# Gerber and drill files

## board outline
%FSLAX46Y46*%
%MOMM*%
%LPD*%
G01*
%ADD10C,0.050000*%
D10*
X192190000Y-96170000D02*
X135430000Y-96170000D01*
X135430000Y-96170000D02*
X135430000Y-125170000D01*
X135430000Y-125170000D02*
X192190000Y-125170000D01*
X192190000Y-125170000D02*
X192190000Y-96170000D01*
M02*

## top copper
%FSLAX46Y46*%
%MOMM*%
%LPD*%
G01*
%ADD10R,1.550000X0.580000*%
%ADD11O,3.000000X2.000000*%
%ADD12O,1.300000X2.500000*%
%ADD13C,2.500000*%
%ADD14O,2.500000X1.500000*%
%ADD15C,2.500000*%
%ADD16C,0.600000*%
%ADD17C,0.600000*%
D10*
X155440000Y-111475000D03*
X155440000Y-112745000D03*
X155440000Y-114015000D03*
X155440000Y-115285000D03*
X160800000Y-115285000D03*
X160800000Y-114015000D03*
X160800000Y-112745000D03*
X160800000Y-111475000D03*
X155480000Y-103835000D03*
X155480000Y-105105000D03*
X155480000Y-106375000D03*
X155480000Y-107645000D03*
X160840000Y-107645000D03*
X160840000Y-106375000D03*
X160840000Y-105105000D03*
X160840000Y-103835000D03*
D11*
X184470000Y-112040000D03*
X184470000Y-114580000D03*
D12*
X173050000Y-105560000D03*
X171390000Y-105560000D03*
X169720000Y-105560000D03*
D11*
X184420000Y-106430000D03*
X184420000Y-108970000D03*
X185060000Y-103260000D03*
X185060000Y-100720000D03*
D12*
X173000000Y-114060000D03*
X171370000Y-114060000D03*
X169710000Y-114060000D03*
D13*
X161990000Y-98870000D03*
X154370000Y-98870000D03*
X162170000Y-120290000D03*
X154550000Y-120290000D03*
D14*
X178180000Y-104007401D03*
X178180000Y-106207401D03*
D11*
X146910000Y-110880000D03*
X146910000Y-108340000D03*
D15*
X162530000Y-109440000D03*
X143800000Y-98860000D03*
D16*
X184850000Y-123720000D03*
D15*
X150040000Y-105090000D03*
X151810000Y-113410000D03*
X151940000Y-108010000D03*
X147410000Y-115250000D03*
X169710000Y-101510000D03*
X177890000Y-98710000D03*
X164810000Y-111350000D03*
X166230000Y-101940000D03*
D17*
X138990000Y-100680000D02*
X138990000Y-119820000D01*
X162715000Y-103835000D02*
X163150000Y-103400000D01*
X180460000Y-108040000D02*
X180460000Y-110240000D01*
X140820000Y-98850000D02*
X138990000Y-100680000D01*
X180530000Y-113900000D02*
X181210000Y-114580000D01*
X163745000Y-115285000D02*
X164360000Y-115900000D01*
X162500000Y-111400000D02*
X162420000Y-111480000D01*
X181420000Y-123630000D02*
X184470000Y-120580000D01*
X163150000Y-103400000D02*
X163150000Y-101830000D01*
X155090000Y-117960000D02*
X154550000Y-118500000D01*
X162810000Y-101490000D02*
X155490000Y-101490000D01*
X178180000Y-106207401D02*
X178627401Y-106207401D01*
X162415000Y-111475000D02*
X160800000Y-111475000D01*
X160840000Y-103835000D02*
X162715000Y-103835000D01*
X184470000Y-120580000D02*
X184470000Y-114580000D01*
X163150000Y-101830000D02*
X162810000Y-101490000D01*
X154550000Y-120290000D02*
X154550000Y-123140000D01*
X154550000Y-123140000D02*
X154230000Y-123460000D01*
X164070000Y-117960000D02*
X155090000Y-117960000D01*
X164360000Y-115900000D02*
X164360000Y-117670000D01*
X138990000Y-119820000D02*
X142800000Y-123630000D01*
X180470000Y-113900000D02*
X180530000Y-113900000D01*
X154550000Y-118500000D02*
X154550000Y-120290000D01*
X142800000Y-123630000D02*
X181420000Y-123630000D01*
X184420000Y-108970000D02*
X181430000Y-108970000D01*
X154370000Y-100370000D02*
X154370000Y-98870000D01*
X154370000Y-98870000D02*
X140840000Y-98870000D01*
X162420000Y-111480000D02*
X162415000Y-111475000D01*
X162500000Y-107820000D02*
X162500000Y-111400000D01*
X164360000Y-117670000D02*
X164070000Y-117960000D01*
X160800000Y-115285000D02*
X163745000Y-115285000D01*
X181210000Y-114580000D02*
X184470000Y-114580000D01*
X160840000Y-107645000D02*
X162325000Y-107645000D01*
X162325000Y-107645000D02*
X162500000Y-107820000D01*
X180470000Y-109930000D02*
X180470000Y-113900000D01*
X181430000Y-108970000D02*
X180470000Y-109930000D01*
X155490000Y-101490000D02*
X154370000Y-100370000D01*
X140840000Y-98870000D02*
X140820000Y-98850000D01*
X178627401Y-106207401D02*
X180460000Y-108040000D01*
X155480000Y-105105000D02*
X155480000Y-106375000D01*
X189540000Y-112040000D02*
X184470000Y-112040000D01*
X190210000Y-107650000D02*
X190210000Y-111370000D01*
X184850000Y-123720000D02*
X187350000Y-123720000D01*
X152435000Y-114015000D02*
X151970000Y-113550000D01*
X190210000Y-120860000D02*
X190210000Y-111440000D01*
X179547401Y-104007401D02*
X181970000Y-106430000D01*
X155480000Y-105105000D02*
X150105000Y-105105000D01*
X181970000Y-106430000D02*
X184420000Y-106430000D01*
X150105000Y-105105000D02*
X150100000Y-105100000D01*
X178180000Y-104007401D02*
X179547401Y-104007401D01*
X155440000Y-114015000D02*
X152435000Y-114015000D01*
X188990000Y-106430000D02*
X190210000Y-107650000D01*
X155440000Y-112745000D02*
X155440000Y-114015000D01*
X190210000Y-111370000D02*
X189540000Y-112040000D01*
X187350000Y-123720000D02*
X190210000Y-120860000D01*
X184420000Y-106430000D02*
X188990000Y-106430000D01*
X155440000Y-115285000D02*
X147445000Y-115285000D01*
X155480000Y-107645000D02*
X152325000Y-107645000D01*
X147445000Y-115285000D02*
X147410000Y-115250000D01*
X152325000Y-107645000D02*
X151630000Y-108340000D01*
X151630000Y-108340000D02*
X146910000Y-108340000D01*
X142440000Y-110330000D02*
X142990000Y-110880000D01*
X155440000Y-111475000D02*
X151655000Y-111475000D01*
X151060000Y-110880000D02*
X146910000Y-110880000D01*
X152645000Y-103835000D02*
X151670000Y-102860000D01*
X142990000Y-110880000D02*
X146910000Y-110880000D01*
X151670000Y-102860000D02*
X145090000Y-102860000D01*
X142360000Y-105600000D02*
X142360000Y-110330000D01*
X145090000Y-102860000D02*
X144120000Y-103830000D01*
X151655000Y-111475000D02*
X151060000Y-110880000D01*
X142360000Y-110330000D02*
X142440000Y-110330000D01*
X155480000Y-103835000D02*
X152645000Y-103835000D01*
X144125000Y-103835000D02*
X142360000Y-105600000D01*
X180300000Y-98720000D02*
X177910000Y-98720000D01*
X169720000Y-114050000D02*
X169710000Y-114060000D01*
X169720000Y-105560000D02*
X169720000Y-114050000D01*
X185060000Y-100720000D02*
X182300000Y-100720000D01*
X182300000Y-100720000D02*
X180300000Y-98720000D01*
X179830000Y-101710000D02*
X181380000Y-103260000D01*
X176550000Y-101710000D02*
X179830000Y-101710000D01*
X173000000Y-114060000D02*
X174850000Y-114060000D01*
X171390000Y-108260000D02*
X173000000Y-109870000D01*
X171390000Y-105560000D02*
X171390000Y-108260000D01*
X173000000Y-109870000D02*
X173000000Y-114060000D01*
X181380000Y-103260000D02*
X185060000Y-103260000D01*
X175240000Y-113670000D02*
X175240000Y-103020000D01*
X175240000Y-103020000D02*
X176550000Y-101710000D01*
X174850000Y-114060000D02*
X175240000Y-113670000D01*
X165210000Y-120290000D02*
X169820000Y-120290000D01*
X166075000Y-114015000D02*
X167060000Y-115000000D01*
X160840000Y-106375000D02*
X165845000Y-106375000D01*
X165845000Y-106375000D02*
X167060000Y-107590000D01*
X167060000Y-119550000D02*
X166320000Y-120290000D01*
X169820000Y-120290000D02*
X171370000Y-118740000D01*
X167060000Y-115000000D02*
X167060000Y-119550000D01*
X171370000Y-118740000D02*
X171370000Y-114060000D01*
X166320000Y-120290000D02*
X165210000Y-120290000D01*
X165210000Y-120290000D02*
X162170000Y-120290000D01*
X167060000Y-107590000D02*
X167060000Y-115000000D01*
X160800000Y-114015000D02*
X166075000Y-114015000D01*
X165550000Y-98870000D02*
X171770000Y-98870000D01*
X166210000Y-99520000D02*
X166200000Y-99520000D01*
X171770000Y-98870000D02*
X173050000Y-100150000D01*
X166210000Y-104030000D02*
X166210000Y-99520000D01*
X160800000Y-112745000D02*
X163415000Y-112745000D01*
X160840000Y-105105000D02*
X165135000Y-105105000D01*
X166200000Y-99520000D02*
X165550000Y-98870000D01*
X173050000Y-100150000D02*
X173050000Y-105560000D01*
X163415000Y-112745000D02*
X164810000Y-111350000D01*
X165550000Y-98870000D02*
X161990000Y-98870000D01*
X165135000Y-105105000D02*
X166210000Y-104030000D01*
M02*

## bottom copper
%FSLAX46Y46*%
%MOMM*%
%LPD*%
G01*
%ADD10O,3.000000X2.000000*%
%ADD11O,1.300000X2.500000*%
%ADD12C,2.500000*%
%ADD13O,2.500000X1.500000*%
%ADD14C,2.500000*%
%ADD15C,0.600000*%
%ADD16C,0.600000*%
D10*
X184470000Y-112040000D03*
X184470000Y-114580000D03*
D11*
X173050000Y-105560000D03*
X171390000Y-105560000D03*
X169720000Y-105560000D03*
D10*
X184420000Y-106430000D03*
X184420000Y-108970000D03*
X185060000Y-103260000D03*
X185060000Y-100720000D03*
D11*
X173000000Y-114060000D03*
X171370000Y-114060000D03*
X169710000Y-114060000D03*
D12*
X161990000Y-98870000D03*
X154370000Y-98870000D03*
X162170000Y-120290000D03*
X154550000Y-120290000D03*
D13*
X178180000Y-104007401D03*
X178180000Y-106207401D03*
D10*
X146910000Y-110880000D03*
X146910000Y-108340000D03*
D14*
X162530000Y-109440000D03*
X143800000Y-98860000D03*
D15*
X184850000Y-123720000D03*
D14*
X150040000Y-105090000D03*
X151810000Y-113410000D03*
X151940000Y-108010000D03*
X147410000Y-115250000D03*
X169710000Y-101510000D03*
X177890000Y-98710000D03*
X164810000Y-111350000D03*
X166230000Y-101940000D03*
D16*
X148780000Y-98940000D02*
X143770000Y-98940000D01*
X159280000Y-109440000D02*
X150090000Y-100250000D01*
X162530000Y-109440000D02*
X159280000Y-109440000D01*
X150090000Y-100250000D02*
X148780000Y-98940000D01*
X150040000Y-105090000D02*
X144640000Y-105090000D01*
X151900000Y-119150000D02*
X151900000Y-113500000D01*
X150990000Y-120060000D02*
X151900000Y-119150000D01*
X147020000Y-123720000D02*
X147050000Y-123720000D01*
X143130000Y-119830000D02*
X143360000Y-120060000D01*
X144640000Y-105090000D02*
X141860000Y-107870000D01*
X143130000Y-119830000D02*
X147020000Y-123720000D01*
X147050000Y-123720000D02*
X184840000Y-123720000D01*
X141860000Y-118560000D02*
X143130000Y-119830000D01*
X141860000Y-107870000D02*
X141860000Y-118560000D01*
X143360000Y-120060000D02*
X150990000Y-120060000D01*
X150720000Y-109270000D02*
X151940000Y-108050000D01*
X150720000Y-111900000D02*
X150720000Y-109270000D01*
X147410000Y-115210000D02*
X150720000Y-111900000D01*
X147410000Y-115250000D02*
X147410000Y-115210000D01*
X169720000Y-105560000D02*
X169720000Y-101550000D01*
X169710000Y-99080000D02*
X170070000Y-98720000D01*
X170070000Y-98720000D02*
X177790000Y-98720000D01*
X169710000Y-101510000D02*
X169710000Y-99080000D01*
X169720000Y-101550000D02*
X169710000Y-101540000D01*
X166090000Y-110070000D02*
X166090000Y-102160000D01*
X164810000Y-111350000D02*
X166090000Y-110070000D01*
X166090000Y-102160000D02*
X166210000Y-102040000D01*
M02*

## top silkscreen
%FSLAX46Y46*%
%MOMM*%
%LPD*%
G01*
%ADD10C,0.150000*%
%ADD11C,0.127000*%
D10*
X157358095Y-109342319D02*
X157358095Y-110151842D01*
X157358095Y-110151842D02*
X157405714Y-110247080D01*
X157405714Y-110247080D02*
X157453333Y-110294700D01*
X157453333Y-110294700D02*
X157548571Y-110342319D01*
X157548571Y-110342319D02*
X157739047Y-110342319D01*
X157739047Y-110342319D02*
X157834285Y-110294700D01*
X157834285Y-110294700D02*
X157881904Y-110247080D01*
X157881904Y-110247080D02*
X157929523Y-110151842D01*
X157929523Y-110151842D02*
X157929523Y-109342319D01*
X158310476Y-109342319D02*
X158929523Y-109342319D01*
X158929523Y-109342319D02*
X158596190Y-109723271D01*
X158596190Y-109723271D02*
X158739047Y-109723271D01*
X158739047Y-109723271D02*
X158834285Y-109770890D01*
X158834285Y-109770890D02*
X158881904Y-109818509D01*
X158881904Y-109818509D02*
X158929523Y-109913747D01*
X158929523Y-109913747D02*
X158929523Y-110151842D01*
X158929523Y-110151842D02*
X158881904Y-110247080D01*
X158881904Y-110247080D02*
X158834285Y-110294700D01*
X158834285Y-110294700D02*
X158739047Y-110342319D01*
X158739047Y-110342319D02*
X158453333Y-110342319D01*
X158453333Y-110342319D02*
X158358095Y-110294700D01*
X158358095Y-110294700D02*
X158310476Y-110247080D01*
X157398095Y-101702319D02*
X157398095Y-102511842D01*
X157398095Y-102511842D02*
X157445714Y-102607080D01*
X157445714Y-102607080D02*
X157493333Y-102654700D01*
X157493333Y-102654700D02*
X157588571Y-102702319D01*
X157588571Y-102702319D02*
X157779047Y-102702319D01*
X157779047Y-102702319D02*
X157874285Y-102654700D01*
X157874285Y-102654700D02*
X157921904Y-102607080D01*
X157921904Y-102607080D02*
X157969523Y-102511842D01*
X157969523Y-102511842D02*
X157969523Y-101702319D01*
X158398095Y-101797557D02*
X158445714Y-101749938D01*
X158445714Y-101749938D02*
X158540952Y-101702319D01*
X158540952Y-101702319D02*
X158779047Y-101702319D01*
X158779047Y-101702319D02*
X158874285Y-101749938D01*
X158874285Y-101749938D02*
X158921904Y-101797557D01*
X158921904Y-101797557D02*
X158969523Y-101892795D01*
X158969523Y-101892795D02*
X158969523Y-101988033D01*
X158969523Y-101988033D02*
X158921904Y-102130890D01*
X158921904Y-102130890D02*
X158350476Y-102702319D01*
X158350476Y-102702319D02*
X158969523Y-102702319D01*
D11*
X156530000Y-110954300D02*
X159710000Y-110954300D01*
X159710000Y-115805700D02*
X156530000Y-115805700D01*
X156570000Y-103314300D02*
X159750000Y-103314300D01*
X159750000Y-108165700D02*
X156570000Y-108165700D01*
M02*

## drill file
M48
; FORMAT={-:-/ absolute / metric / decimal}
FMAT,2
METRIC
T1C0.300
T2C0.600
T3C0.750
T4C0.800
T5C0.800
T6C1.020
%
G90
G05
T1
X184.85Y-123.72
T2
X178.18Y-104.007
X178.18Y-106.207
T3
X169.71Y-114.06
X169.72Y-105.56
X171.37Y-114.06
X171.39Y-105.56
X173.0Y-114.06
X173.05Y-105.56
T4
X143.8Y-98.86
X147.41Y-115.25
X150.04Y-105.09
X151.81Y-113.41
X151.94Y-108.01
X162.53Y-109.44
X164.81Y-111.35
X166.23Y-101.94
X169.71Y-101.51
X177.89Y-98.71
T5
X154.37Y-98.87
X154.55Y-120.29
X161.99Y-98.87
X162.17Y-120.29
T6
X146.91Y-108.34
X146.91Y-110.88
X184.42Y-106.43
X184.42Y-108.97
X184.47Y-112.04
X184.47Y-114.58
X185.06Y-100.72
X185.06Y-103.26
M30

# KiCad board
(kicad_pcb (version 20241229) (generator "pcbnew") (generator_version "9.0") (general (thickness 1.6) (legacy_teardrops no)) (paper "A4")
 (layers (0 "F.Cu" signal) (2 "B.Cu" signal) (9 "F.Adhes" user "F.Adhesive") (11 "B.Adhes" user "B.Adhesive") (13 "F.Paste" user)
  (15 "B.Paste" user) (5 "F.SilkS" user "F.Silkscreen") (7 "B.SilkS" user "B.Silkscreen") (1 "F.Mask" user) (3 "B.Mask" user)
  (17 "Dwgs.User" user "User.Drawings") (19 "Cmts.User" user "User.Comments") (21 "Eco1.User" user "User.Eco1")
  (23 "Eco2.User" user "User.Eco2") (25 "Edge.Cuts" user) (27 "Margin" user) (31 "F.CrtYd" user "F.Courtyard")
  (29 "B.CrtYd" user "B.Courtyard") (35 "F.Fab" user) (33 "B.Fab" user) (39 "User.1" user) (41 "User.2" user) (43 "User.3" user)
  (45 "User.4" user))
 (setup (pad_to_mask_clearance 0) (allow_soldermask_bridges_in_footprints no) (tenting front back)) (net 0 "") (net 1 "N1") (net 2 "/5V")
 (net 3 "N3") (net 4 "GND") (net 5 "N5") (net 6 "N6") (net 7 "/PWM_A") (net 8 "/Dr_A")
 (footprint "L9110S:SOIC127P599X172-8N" (layer "F.Cu") (at 158.12 113.38)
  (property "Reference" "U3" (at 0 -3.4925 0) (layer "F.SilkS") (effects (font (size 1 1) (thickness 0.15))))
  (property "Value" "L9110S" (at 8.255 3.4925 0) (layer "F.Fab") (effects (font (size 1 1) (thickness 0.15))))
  (fp_line (start -1.59 -2.4257) (end 1.59 -2.4257) (stroke (width 0.127) (type solid)) (layer "F.SilkS"))
  (fp_line (start 1.59 2.4257) (end -1.59 2.4257) (stroke (width 0.127) (type solid)) (layer "F.SilkS"))
  (pad "1" smd rect (at -2.68 -1.905) (size 1.55 0.58) (layers "F.Cu" "F.Mask" "F.Paste") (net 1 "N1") (solder_mask_margin 0.102))
  (pad "2" smd rect (at -2.68 -0.635) (size 1.55 0.58) (layers "F.Cu" "F.Mask" "F.Paste") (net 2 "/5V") (solder_mask_margin 0.102))
  (pad "3" smd rect (at -2.68 0.635) (size 1.55 0.58) (layers "F.Cu" "F.Mask" "F.Paste") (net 2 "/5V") (solder_mask_margin 0.102))
  (pad "4" smd rect (at -2.68 1.905) (size 1.55 0.58) (layers "F.Cu" "F.Mask" "F.Paste") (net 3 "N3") (solder_mask_margin 0.102))
  (pad "5" smd rect (at 2.68 1.905) (size 1.55 0.58) (layers "F.Cu" "F.Mask" "F.Paste") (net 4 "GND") (solder_mask_margin 0.102))
  (pad "6" smd rect (at 2.68 0.635) (size 1.55 0.58) (layers "F.Cu" "F.Mask" "F.Paste") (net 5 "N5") (solder_mask_margin 0.102))
  (pad "7" smd rect (at 2.68 -0.635) (size 1.55 0.58) (layers "F.Cu" "F.Mask" "F.Paste") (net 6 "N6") (solder_mask_margin 0.102))
  (pad "8" smd rect (at 2.68 -1.905) (size 1.55 0.58) (layers "F.Cu" "F.Mask" "F.Paste") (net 4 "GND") (solder_mask_margin 0.102)))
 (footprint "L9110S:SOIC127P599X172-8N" (layer "F.Cu") (at 158.16 105.74)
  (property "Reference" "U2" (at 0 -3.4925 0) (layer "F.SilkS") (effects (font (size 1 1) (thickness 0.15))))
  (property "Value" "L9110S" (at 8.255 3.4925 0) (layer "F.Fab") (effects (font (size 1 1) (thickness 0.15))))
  (fp_line (start -1.59 -2.4257) (end 1.59 -2.4257) (stroke (width 0.127) (type solid)) (layer "F.SilkS"))
  (fp_line (start 1.59 2.4257) (end -1.59 2.4257) (stroke (width 0.127) (type solid)) (layer "F.SilkS"))
  (pad "1" smd rect (at -2.68 -1.905) (size 1.55 0.58) (layers "F.Cu" "F.Mask" "F.Paste") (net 1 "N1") (solder_mask_margin 0.102))
  (pad "2" smd rect (at -2.68 -0.635) (size 1.55 0.58) (layers "F.Cu" "F.Mask" "F.Paste") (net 2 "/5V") (solder_mask_margin 0.102))
  (pad "3" smd rect (at -2.68 0.635) (size 1.55 0.58) (layers "F.Cu" "F.Mask" "F.Paste") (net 2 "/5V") (solder_mask_margin 0.102))
  (pad "4" smd rect (at -2.68 1.905) (size 1.55 0.58) (layers "F.Cu" "F.Mask" "F.Paste") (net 3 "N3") (solder_mask_margin 0.102))
  (pad "5" smd rect (at 2.68 1.905) (size 1.55 0.58) (layers "F.Cu" "F.Mask" "F.Paste") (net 4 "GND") (solder_mask_margin 0.102))
  (pad "6" smd rect (at 2.68 0.635) (size 1.55 0.58) (layers "F.Cu" "F.Mask" "F.Paste") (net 5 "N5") (solder_mask_margin 0.102))
  (pad "7" smd rect (at 2.68 -0.635) (size 1.55 0.58) (layers "F.Cu" "F.Mask" "F.Paste") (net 6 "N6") (solder_mask_margin 0.102))
  (pad "8" smd rect (at 2.68 -1.905) (size 1.55 0.58) (layers "F.Cu" "F.Mask" "F.Paste") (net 4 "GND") (solder_mask_margin 0.102)))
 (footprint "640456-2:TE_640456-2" (layer "B.Cu") (at 184.47 112.04 90)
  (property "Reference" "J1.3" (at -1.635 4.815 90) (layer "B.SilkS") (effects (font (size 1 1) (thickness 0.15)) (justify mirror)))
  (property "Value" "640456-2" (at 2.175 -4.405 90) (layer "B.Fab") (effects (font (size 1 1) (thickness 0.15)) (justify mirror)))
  (pad "1" thru_hole oval (at 0 0 90) (size 2 3) (drill 1.02) (layers "*.Cu" "*.Mask") (remove_unused_layers no) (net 2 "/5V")
   (solder_mask_margin 0.102))
  (pad "2" thru_hole oval (at -2.54 0 90) (size 2 3) (drill 1.02) (layers "*.Cu" "*.Mask") (remove_unused_layers no) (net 4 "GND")
   (solder_mask_margin 0.102)))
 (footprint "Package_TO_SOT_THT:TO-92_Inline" (layer "B.Cu") (at 172.66 105.54 180)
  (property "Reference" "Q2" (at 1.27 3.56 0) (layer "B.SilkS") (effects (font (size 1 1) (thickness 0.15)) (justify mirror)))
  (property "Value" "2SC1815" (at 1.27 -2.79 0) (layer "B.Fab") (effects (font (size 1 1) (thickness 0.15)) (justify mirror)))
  (pad "1" thru_hole oval (at -0.39 -0.02 180) (size 1.3 2.5) (drill 0.75) (layers "*.Cu" "*.Mask") (remove_unused_layers no) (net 6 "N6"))
  (pad "2" thru_hole oval (at 1.27 -0.02 180) (size 1.3 2.5) (drill 0.75) (layers "*.Cu" "*.Mask") (remove_unused_layers no)
   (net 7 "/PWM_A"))
  (pad "3" thru_hole oval (at 2.94 -0.02 180) (size 1.3 2.5) (drill 0.75) (layers "*.Cu" "*.Mask") (remove_unused_layers no) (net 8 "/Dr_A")))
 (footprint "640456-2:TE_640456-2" (layer "B.Cu") (at 184.42 106.43 90)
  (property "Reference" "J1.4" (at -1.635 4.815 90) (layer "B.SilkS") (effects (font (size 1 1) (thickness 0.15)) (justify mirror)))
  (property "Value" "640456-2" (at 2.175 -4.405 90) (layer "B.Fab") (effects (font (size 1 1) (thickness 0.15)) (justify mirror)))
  (pad "1" thru_hole oval (at 0 0 90) (size 2 3) (drill 1.02) (layers "*.Cu" "*.Mask") (remove_unused_layers no) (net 2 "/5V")
   (solder_mask_margin 0.102))
  (pad "2" thru_hole oval (at -2.54 0 90) (size 2 3) (drill 1.02) (layers "*.Cu" "*.Mask") (remove_unused_layers no) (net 4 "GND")
   (solder_mask_margin 0.102)))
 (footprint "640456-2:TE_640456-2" (layer "B.Cu") (at 185.06 103.26 -90)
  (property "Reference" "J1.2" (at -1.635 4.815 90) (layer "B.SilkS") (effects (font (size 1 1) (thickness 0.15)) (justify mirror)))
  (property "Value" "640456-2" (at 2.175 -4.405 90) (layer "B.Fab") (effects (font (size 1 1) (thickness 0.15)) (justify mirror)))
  (pad "1" thru_hole oval (at 0 0 270) (size 2 3) (drill 1.02) (layers "*.Cu" "*.Mask") (remove_unused_layers no) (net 7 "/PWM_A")
   (solder_mask_margin 0.102))
  (pad "2" thru_hole oval (at -2.54 0 270) (size 2 3) (drill 1.02) (layers "*.Cu" "*.Mask") (remove_unused_layers no) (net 8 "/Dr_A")
   (solder_mask_margin 0.102)))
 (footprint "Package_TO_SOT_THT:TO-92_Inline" (layer "B.Cu") (at 172.64 114.06 180)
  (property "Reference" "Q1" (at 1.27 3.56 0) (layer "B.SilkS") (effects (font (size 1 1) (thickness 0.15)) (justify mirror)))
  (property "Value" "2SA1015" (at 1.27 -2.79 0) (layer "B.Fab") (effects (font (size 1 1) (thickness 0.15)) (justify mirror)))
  (pad "1" thru_hole oval (at -0.36 0 180) (size 1.3 2.5) (drill 0.75) (layers "*.Cu" "*.Mask") (remove_unused_layers no) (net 7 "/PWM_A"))
  (pad "2" thru_hole oval (at 1.27 0 180) (size 1.3 2.5) (drill 0.75) (layers "*.Cu" "*.Mask") (remove_unused_layers no) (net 5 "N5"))
  (pad "3" thru_hole oval (at 2.93 0 180) (size 1.3 2.5) (drill 0.75) (layers "*.Cu" "*.Mask") (remove_unused_layers no) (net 8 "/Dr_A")))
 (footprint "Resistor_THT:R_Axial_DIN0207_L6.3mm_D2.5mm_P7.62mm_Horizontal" (layer "B.Cu") (at 161.99 98.87 180)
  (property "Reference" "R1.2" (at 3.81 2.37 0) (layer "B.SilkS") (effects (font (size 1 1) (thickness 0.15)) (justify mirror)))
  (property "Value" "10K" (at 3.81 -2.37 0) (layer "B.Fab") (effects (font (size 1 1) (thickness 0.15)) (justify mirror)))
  (pad "1" thru_hole circle (at 0 0 180) (size 2.5 2.5) (drill 0.8) (layers "*.Cu" "*.Mask") (remove_unused_layers no) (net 6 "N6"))
  (pad "2" thru_hole circle (at 7.62 0 180) (size 2.5 2.5) (drill 0.8) (layers "*.Cu" "*.Mask") (remove_unused_layers no) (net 4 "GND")))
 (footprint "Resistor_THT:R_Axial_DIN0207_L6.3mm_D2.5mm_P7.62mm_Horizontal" (layer "B.Cu") (at 162.17 120.29 180)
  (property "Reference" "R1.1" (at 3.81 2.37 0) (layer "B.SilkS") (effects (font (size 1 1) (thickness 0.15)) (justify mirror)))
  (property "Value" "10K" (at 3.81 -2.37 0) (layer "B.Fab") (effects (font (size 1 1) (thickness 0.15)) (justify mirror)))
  (pad "1" thru_hole circle (at 0 0 180) (size 2.5 2.5) (drill 0.8) (layers "*.Cu" "*.Mask") (remove_unused_layers no) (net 5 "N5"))
  (pad "2" thru_hole circle (at 7.62 0 180) (size 2.5 2.5) (drill 0.8) (layers "*.Cu" "*.Mask") (remove_unused_layers no) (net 4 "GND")))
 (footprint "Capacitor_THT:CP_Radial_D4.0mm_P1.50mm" (layer "B.Cu") (at 178.18 104.337401 -90)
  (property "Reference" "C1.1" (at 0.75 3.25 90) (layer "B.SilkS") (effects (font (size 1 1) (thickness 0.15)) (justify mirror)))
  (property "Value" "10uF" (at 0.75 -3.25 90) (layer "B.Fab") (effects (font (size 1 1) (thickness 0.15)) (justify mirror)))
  (pad "1" thru_hole oval (at -0.33 0 270) (size 1.5 2.5) (drill 0.6) (layers "*.Cu" "*.Mask") (remove_unused_layers no) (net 2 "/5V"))
  (pad "2" thru_hole oval (at 1.87 0 270) (size 1.5 2.5) (drill 0.6) (layers "*.Cu" "*.Mask") (remove_unused_layers no) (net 4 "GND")))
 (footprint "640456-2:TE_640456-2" (layer "B.Cu") (at 146.91 110.88 -90)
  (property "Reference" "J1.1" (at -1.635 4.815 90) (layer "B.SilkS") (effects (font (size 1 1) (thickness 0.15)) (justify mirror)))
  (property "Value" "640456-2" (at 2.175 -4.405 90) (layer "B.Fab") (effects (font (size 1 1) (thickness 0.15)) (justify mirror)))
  (pad "1" thru_hole oval (at 0 0 270) (size 2 3) (drill 1.02) (layers "*.Cu" "*.Mask") (remove_unused_layers no) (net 1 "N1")
   (solder_mask_margin 0.102))
  (pad "2" thru_hole oval (at -2.54 0 270) (size 2 3) (drill 1.02) (layers "*.Cu" "*.Mask") (remove_unused_layers no) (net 3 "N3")
   (solder_mask_margin 0.102)))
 (gr_line (start 192.19 96.17) (end 135.43 96.17) (stroke (width 0.05) (type default)) (layer "Edge.Cuts"))
 (gr_line (start 135.43 96.17) (end 135.43 125.17) (stroke (width 0.05) (type default)) (layer "Edge.Cuts"))
 (gr_line (start 135.43 125.17) (end 192.19 125.17) (stroke (width 0.05) (type default)) (layer "Edge.Cuts"))
 (gr_line (start 192.19 125.17) (end 192.19 96.17) (stroke (width 0.05) (type default)) (layer "Edge.Cuts"))
 (segment (start 138.99 100.68) (end 138.99 119.82) (width 0.6) (layer "F.Cu") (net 4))
 (segment (start 162.715 103.835) (end 163.15 103.4) (width 0.6) (layer "F.Cu") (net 4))
 (segment (start 180.46 108.04) (end 180.46 110.24) (width 0.6) (layer "F.Cu") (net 4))
 (segment (start 140.82 98.85) (end 138.99 100.68) (width 0.6) (layer "F.Cu") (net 4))
 (segment (start 180.53 113.9) (end 181.21 114.58) (width 0.6) (layer "F.Cu") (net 4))
 (segment (start 163.745 115.285) (end 164.36 115.9) (width 0.6) (layer "F.Cu") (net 4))
 (segment (start 162.5 111.4) (end 162.42 111.48) (width 0.6) (layer "F.Cu") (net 4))
 (segment (start 181.42 123.63) (end 184.47 120.58) (width 0.6) (layer "F.Cu") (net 4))
 (segment (start 163.15 103.4) (end 163.15 101.83) (width 0.6) (layer "F.Cu") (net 4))
 (segment (start 155.09 117.96) (end 154.55 118.5) (width 0.6) (layer "F.Cu") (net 4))
 (segment (start 162.81 101.49) (end 155.49 101.49) (width 0.6) (layer "F.Cu") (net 4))
 (segment (start 178.18 106.207401) (end 178.627401 106.207401) (width 0.6) (layer "F.Cu") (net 4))
 (segment (start 162.415 111.475) (end 160.8 111.475) (width 0.6) (layer "F.Cu") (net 4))
 (segment (start 160.84 103.835) (end 162.715 103.835) (width 0.6) (layer "F.Cu") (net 4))
 (segment (start 184.47 120.58) (end 184.47 114.58) (width 0.6) (layer "F.Cu") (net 4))
 (segment (start 163.15 101.83) (end 162.81 101.49) (width 0.6) (layer "F.Cu") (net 4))
 (segment (start 154.55 120.29) (end 154.55 123.14) (width 0.6) (layer "F.Cu") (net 4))
 (segment (start 154.55 123.14) (end 154.23 123.46) (width 0.6) (layer "F.Cu") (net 4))
 (segment (start 164.07 117.96) (end 155.09 117.96) (width 0.6) (layer "F.Cu") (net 4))
 (segment (start 164.36 115.9) (end 164.36 117.67) (width 0.6) (layer "F.Cu") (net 4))
 (segment (start 138.99 119.82) (end 142.8 123.63) (width 0.6) (layer "F.Cu") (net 4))
 (segment (start 180.47 113.9) (end 180.53 113.9) (width 0.6) (layer "F.Cu") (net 4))
 (segment (start 154.55 118.5) (end 154.55 120.29) (width 0.6) (layer "F.Cu") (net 4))
 (segment (start 142.8 123.63) (end 181.42 123.63) (width 0.6) (layer "F.Cu") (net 4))
 (segment (start 184.42 108.97) (end 181.43 108.97) (width 0.6) (layer "F.Cu") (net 4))
 (segment (start 154.37 100.37) (end 154.37 98.87) (width 0.6) (layer "F.Cu") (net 4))
 (segment (start 154.37 98.87) (end 140.84 98.87) (width 0.6) (layer "F.Cu") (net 4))
 (segment (start 162.42 111.48) (end 162.415 111.475) (width 0.6) (layer "F.Cu") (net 4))
 (segment (start 162.5 107.82) (end 162.5 111.4) (width 0.6) (layer "F.Cu") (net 4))
 (segment (start 164.36 117.67) (end 164.07 117.96) (width 0.6) (layer "F.Cu") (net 4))
 (segment (start 160.8 115.285) (end 163.745 115.285) (width 0.6) (layer "F.Cu") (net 4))
 (segment (start 181.21 114.58) (end 184.47 114.58) (width 0.6) (layer "F.Cu") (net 4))
 (segment (start 160.84 107.645) (end 162.325 107.645) (width 0.6) (layer "F.Cu") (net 4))
 (segment (start 162.325 107.645) (end 162.5 107.82) (width 0.6) (layer "F.Cu") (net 4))
 (segment (start 180.47 109.93) (end 180.47 113.9) (width 0.6) (layer "F.Cu") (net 4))
 (segment (start 181.43 108.97) (end 180.47 109.93) (width 0.6) (layer "F.Cu") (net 4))
 (segment (start 155.49 101.49) (end 154.37 100.37) (width 0.6) (layer "F.Cu") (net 4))
 (segment (start 140.84 98.87) (end 140.82 98.85) (width 0.6) (layer "F.Cu") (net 4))
 (segment (start 178.627401 106.207401) (end 180.46 108.04) (width 0.6) (layer "F.Cu") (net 4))
 (via (at 162.53 109.44) (size 2.5) (drill 0.8) (layers "F.Cu" "B.Cu") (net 4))
 (via (at 143.8 98.86) (size 2.5) (drill 0.8) (layers "F.Cu" "B.Cu") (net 4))
 (segment (start 148.78 98.94) (end 143.77 98.94) (width 0.6) (layer "B.Cu") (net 4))
 (segment (start 159.28 109.44) (end 150.09 100.25) (width 0.6) (layer "B.Cu") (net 4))
 (segment (start 162.53 109.44) (end 159.28 109.44) (width 0.6) (layer "B.Cu") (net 4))
 (segment (start 150.09 100.25) (end 148.78 98.94) (width 0.6) (layer "B.Cu") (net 4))
 (segment (start 155.48 105.105) (end 155.48 106.375) (width 0.6) (layer "F.Cu") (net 2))
 (segment (start 189.54 112.04) (end 184.47 112.04) (width 0.6) (layer "F.Cu") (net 2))
 (segment (start 190.21 107.65) (end 190.21 111.37) (width 0.6) (layer "F.Cu") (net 2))
 (segment (start 184.85 123.72) (end 187.35 123.72) (width 0.6) (layer "F.Cu") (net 2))
 (segment (start 152.435 114.015) (end 151.97 113.55) (width 0.6) (layer "F.Cu") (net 2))
 (segment (start 190.21 120.86) (end 190.21 111.44) (width 0.6) (layer "F.Cu") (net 2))
 (segment (start 179.547401 104.007401) (end 181.97 106.43) (width 0.6) (layer "F.Cu") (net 2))
 (segment (start 155.48 105.105) (end 150.105 105.105) (width 0.6) (layer "F.Cu") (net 2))
 (segment (start 181.97 106.43) (end 184.42 106.43) (width 0.6) (layer "F.Cu") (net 2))
 (segment (start 150.105 105.105) (end 150.1 105.1) (width 0.6) (layer "F.Cu") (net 2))
 (segment (start 178.18 104.007401) (end 179.547401 104.007401) (width 0.6) (layer "F.Cu") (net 2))
 (segment (start 155.44 114.015) (end 152.435 114.015) (width 0.6) (layer "F.Cu") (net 2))
 (segment (start 188.99 106.43) (end 190.21 107.65) (width 0.6) (layer "F.Cu") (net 2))
 (segment (start 155.44 112.745) (end 155.44 114.015) (width 0.6) (layer "F.Cu") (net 2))
 (segment (start 190.21 111.37) (end 189.54 112.04) (width 0.6) (layer "F.Cu") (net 2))
 (segment (start 187.35 123.72) (end 190.21 120.86) (width 0.6) (layer "F.Cu") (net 2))
 (segment (start 184.42 106.43) (end 188.99 106.43) (width 0.6) (layer "F.Cu") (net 2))
 (via (at 184.85 123.72) (size 0.6) (drill 0.3) (layers "F.Cu" "B.Cu") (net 2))
 (via (at 150.04 105.09) (size 2.5) (drill 0.8) (layers "F.Cu" "B.Cu") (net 2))
 (via (at 151.81 113.41) (size 2.5) (drill 0.8) (layers "F.Cu" "B.Cu") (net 2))
 (segment (start 150.04 105.09) (end 144.64 105.09) (width 0.6) (layer "B.Cu") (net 2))
 (segment (start 151.9 119.15) (end 151.9 113.5) (width 0.6) (layer "B.Cu") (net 2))
 (segment (start 150.99 120.06) (end 151.9 119.15) (width 0.6) (layer "B.Cu") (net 2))
 (segment (start 147.02 123.72) (end 147.05 123.72) (width 0.6) (layer "B.Cu") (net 2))
 (segment (start 143.13 119.83) (end 143.36 120.06) (width 0.6) (layer "B.Cu") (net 2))
 (segment (start 144.64 105.09) (end 141.86 107.87) (width 0.6) (layer "B.Cu") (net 2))
 (segment (start 143.13 119.83) (end 147.02 123.72) (width 0.6) (layer "B.Cu") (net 2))
 (segment (start 147.05 123.72) (end 184.84 123.72) (width 0.6) (layer "B.Cu") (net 2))
 (segment (start 141.86 118.56) (end 143.13 119.83) (width 0.6) (layer "B.Cu") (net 2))
 (segment (start 141.86 107.87) (end 141.86 118.56) (width 0.6) (layer "B.Cu") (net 2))
 (segment (start 143.36 120.06) (end 150.99 120.06) (width 0.6) (layer "B.Cu") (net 2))
 (segment (start 155.44 115.285) (end 147.445 115.285) (width 0.6) (layer "F.Cu") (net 3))
 (segment (start 155.48 107.645) (end 152.325 107.645) (width 0.6) (layer "F.Cu") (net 3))
 (segment (start 147.445 115.285) (end 147.41 115.25) (width 0.6) (layer "F.Cu") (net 3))
 (segment (start 152.325 107.645) (end 151.63 108.34) (width 0.6) (layer "F.Cu") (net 3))
 (segment (start 151.63 108.34) (end 146.91 108.34) (width 0.6) (layer "F.Cu") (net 3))
 (via (at 151.94 108.01) (size 2.5) (drill 0.8) (layers "F.Cu" "B.Cu") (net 3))
 (via (at 147.41 115.25) (size 2.5) (drill 0.8) (layers "F.Cu" "B.Cu") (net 3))
 (segment (start 150.72 109.27) (end 151.94 108.05) (width 0.6) (layer "B.Cu") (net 3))
 (segment (start 150.72 111.9) (end 150.72 109.27) (width 0.6) (layer "B.Cu") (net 3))
 (segment (start 147.41 115.21) (end 150.72 111.9) (width 0.6) (layer "B.Cu") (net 3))
 (segment (start 147.41 115.25) (end 147.41 115.21) (width 0.6) (layer "B.Cu") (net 3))
 (segment (start 142.44 110.33) (end 142.99 110.88) (width 0.6) (layer "F.Cu") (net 1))
 (segment (start 155.44 111.475) (end 151.655 111.475) (width 0.6) (layer "F.Cu") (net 1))
 (segment (start 151.06 110.88) (end 146.91 110.88) (width 0.6) (layer "F.Cu") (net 1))
 (segment (start 152.645 103.835) (end 151.67 102.86) (width 0.6) (layer "F.Cu") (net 1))
 (segment (start 142.99 110.88) (end 146.91 110.88) (width 0.6) (layer "F.Cu") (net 1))
 (segment (start 151.67 102.86) (end 145.09 102.86) (width 0.6) (layer "F.Cu") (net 1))
 (segment (start 142.36 105.6) (end 142.36 110.33) (width 0.6) (layer "F.Cu") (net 1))
 (segment (start 145.09 102.86) (end 144.12 103.83) (width 0.6) (layer "F.Cu") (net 1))
 (segment (start 151.655 111.475) (end 151.06 110.88) (width 0.6) (layer "F.Cu") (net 1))
 (segment (start 142.36 110.33) (end 142.44 110.33) (width 0.6) (layer "F.Cu") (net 1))
 (segment (start 155.48 103.835) (end 152.645 103.835) (width 0.6) (layer "F.Cu") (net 1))
 (segment (start 144.125 103.835) (end 142.36 105.6) (width 0.6) (layer "F.Cu") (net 1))
 (segment (start 180.3 98.72) (end 177.91 98.72) (width 0.6) (layer "F.Cu") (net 8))
 (segment (start 169.72 114.05) (end 169.71 114.06) (width 0.6) (layer "F.Cu") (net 8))
 (segment (start 169.72 105.56) (end 169.72 114.05) (width 0.6) (layer "F.Cu") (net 8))
 (segment (start 185.06 100.72) (end 182.3 100.72) (width 0.6) (layer "F.Cu") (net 8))
 (segment (start 182.3 100.72) (end 180.3 98.72) (width 0.6) (layer "F.Cu") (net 8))
 (via (at 169.71 101.51) (size 2.5) (drill 0.8) (layers "F.Cu" "B.Cu") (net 8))
 (via (at 177.89 98.71) (size 2.5) (drill 0.8) (layers "F.Cu" "B.Cu") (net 8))
 (segment (start 169.72 105.56) (end 169.72 101.55) (width 0.6) (layer "B.Cu") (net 8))
 (segment (start 169.71 99.08) (end 170.07 98.72) (width 0.6) (layer "B.Cu") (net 8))
 (segment (start 170.07 98.72) (end 177.79 98.72) (width 0.6) (layer "B.Cu") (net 8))
 (segment (start 169.71 101.51) (end 169.71 99.08) (width 0.6) (layer "B.Cu") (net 8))
 (segment (start 169.72 101.55) (end 169.71 101.54) (width 0.6) (layer "B.Cu") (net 8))
 (segment (start 179.83 101.71) (end 181.38 103.26) (width 0.6) (layer "F.Cu") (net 7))
 (segment (start 176.55 101.71) (end 179.83 101.71) (width 0.6) (layer "F.Cu") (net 7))
 (segment (start 173 114.06) (end 174.85 114.06) (width 0.6) (layer "F.Cu") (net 7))
 (segment (start 171.39 108.26) (end 173 109.87) (width 0.6) (layer "F.Cu") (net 7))
 (segment (start 171.39 105.56) (end 171.39 108.26) (width 0.6) (layer "F.Cu") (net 7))
 (segment (start 173 109.87) (end 173 114.06) (width 0.6) (layer "F.Cu") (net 7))
 (segment (start 181.38 103.26) (end 185.06 103.26) (width 0.6) (layer "F.Cu") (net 7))
 (segment (start 175.24 113.67) (end 175.24 103.02) (width 0.6) (layer "F.Cu") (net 7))
 (segment (start 175.24 103.02) (end 176.55 101.71) (width 0.6) (layer "F.Cu") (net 7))
 (segment (start 174.85 114.06) (end 175.24 113.67) (width 0.6) (layer "F.Cu") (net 7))
 (segment (start 165.21 120.29) (end 169.82 120.29) (width 0.6) (layer "F.Cu") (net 5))
 (segment (start 166.075 114.015) (end 167.06 115) (width 0.6) (layer "F.Cu") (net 5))
 (segment (start 160.84 106.375) (end 165.845 106.375) (width 0.6) (layer "F.Cu") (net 5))
 (segment (start 165.845 106.375) (end 167.06 107.59) (width 0.6) (layer "F.Cu") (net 5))
 (segment (start 167.06 119.55) (end 166.32 120.29) (width 0.6) (layer "F.Cu") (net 5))
 (segment (start 169.82 120.29) (end 171.37 118.74) (width 0.6) (layer "F.Cu") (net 5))
 (segment (start 167.06 115) (end 167.06 119.55) (width 0.6) (layer "F.Cu") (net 5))
 (segment (start 171.37 118.74) (end 171.37 114.06) (width 0.6) (layer "F.Cu") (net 5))
 (segment (start 166.32 120.29) (end 165.21 120.29) (width 0.6) (layer "F.Cu") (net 5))
 (segment (start 165.21 120.29) (end 162.17 120.29) (width 0.6) (layer "F.Cu") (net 5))
 (segment (start 167.06 107.59) (end 167.06 115) (width 0.6) (layer "F.Cu") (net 5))
 (segment (start 160.8 114.015) (end 166.075 114.015) (width 0.6) (layer "F.Cu") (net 5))
 (segment (start 165.55 98.87) (end 171.77 98.87) (width 0.6) (layer "F.Cu") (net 6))
 (segment (start 166.21 99.52) (end 166.2 99.52) (width 0.6) (layer "F.Cu") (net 6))
 (segment (start 171.77 98.87) (end 173.05 100.15) (width 0.6) (layer "F.Cu") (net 6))
 (segment (start 166.21 104.03) (end 166.21 99.52) (width 0.6) (layer "F.Cu") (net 6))
 (segment (start 160.8 112.745) (end 163.415 112.745) (width 0.6) (layer "F.Cu") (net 6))
 (segment (start 160.84 105.105) (end 165.135 105.105) (width 0.6) (layer "F.Cu") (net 6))
 (segment (start 166.2 99.52) (end 165.55 98.87) (width 0.6) (layer "F.Cu") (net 6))
 (segment (start 173.05 100.15) (end 173.05 105.56) (width 0.6) (layer "F.Cu") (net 6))
 (segment (start 163.415 112.745) (end 164.81 111.35) (width 0.6) (layer "F.Cu") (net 6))
 (segment (start 165.55 98.87) (end 161.99 98.87) (width 0.6) (layer "F.Cu") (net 6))
 (segment (start 165.135 105.105) (end 166.21 104.03) (width 0.6) (layer "F.Cu") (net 6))
 (via (at 164.81 111.35) (size 2.5) (drill 0.8) (layers "F.Cu" "B.Cu") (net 6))
 (via (at 166.23 101.94) (size 2.5) (drill 0.8) (layers "F.Cu" "B.Cu") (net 6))
 (segment (start 166.09 110.07) (end 166.09 102.16) (width 0.6) (layer "B.Cu") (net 6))
 (segment (start 164.81 111.35) (end 166.09 110.07) (width 0.6) (layer "B.Cu") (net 6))
 (segment (start 166.09 102.16) (end 166.21 102.04) (width 0.6) (layer "B.Cu") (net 6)))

